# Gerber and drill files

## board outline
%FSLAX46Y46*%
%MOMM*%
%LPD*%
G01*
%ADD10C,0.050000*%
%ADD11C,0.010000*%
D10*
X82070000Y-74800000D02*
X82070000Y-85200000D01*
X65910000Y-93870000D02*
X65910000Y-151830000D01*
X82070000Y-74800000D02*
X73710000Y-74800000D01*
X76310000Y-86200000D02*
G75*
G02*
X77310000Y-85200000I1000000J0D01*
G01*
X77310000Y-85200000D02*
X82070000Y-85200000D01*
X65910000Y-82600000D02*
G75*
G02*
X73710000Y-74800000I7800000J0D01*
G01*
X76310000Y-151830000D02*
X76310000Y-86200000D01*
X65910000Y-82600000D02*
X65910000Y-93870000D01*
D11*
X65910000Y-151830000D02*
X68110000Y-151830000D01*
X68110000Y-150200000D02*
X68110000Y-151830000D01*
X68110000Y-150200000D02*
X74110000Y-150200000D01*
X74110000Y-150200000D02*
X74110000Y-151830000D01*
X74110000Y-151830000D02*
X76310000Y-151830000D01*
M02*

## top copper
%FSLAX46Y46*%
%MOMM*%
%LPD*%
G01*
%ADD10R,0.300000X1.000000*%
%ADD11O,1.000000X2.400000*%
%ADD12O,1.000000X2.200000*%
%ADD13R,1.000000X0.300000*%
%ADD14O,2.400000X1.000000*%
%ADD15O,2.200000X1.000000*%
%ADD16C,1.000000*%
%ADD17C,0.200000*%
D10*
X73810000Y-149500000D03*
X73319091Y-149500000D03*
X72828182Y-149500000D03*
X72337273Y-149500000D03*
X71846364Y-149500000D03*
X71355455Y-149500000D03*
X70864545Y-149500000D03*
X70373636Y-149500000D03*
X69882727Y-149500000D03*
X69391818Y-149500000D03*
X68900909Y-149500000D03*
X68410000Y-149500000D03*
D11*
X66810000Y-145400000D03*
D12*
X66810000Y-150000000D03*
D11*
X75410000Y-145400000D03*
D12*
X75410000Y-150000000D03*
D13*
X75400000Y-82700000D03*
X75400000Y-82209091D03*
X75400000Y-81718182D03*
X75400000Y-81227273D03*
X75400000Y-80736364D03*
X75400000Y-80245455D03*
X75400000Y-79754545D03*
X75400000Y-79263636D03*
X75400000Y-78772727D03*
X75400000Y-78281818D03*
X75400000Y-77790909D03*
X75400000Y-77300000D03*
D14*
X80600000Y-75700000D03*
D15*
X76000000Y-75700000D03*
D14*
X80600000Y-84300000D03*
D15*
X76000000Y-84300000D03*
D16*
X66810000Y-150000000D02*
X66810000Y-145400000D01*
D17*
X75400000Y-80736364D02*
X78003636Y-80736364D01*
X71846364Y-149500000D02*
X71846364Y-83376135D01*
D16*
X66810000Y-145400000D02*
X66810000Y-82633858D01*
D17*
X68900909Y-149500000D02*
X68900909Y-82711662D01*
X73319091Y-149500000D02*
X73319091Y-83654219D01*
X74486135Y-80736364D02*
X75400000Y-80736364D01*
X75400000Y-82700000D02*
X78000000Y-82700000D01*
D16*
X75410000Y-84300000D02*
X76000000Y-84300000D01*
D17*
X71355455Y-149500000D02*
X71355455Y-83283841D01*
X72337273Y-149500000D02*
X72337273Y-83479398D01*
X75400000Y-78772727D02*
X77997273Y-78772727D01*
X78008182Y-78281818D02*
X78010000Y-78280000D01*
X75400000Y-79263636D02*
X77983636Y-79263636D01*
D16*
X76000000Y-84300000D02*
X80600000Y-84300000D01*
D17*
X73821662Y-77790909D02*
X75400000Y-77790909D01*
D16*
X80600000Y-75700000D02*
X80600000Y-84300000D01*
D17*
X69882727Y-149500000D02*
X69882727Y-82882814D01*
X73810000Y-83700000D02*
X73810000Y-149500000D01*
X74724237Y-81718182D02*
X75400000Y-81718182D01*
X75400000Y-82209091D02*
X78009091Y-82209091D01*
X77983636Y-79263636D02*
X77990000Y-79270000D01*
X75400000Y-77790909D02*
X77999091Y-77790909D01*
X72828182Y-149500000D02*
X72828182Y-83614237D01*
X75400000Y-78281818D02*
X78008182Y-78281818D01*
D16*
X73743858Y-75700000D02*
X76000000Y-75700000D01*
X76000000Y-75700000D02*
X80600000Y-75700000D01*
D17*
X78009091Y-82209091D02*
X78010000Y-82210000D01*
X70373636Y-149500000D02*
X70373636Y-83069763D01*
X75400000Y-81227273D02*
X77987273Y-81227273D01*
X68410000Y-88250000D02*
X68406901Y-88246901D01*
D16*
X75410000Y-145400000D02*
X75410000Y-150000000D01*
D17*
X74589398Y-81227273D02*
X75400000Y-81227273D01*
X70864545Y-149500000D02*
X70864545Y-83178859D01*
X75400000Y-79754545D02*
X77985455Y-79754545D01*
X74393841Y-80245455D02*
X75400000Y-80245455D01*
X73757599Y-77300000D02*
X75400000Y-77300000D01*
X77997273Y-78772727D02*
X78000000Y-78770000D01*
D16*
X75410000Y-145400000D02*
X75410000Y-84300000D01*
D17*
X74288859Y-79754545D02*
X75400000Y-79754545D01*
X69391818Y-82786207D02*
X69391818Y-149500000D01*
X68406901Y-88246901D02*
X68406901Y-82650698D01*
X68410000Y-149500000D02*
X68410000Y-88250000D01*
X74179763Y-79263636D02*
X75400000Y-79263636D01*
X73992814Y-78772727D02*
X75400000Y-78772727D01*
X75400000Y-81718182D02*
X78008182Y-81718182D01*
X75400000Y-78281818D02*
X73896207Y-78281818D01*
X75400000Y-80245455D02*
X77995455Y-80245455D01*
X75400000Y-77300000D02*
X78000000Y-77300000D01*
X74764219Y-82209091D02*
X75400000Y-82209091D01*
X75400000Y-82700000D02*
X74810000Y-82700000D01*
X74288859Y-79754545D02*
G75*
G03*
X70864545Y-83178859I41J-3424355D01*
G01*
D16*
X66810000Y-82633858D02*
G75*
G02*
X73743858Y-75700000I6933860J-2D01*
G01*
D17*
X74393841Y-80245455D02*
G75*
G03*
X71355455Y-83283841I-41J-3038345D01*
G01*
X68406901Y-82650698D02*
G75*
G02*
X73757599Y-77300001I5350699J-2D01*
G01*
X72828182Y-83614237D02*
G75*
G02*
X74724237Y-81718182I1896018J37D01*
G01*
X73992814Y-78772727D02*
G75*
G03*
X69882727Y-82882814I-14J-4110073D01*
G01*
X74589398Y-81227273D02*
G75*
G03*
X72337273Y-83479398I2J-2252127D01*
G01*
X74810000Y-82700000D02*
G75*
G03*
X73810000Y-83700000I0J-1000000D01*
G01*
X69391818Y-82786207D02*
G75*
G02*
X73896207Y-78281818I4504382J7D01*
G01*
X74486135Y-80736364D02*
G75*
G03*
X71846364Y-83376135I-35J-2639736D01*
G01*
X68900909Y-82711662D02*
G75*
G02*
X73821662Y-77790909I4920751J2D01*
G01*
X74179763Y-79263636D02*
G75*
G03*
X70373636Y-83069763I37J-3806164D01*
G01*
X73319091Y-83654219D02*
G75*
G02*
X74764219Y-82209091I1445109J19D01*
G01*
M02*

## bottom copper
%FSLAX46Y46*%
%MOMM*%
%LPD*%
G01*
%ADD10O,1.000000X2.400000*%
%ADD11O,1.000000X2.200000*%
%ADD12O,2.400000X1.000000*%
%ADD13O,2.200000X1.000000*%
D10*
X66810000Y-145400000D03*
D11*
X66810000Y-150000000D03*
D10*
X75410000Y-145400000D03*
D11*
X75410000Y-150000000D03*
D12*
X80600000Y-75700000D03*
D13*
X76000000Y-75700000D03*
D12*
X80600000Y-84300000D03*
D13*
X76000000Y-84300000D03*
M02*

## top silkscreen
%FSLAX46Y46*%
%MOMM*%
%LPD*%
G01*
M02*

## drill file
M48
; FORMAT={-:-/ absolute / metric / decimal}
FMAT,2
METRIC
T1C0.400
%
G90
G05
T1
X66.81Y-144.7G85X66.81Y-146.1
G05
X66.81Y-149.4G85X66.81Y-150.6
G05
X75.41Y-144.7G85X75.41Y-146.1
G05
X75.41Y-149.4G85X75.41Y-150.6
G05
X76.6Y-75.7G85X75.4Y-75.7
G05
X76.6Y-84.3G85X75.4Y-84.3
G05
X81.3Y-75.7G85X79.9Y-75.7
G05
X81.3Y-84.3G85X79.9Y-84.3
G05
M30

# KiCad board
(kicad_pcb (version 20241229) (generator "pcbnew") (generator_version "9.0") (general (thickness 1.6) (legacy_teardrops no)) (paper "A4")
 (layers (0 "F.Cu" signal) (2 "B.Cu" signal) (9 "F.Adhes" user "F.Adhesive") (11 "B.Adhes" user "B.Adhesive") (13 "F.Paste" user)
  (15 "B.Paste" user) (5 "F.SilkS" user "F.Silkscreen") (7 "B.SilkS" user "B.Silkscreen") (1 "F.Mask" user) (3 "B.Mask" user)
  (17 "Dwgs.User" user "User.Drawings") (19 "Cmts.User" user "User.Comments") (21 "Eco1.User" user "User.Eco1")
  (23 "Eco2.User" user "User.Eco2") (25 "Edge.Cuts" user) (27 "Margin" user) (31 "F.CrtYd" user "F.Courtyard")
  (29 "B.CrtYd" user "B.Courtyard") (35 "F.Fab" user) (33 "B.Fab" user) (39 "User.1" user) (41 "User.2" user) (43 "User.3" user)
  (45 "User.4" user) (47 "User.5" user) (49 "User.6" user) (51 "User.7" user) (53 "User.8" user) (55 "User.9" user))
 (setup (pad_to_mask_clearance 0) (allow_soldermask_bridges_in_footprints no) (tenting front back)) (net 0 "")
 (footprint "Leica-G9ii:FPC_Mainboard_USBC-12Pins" (layer "F.Cu") (at 71.11 150)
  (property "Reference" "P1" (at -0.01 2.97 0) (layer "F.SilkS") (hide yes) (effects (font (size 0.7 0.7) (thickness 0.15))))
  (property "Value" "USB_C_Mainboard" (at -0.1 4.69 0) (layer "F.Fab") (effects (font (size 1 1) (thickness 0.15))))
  (fp_line (start -5.2 1.83) (end -3 1.83) (stroke (width 0.01) (type solid)) (layer "Edge.Cuts"))
  (fp_line (start -3 0.2) (end -3 1.83) (stroke (width 0.01) (type solid)) (layer "Edge.Cuts"))
  (fp_line (start -3 0.2) (end 3 0.2) (stroke (width 0.01) (type solid)) (layer "Edge.Cuts"))
  (fp_line (start 3 0.2) (end 3 1.83) (stroke (width 0.01) (type solid)) (layer "Edge.Cuts"))
  (fp_line (start 3 1.83) (end 5.2 1.83) (stroke (width 0.01) (type solid)) (layer "Edge.Cuts"))
  (pad "1" smd rect (at 2.7 -0.5) (size 0.3 1) (layers "F.Cu" "F.Mask" "F.Paste"))
  (pad "2" smd rect (at 2.209091 -0.5) (size 0.3 1) (layers "F.Cu" "F.Mask" "F.Paste"))
  (pad "3" smd rect (at 1.718182 -0.5) (size 0.3 1) (layers "F.Cu" "F.Mask" "F.Paste"))
  (pad "4" smd rect (at 1.227273 -0.5) (size 0.3 1) (layers "F.Cu" "F.Mask" "F.Paste"))
  (pad "5" smd rect (at 0.736364 -0.5) (size 0.3 1) (layers "F.Cu" "F.Mask" "F.Paste"))
  (pad "6" smd rect (at 0.245455 -0.5) (size 0.3 1) (layers "F.Cu" "F.Mask" "F.Paste"))
  (pad "7" smd rect (at -0.245455 -0.5) (size 0.3 1) (layers "F.Cu" "F.Mask" "F.Paste"))
  (pad "8" smd rect (at -0.736364 -0.5) (size 0.3 1) (layers "F.Cu" "F.Mask" "F.Paste"))
  (pad "9" smd rect (at -1.227273 -0.5) (size 0.3 1) (layers "F.Cu" "F.Mask" "F.Paste"))
  (pad "10" smd rect (at -1.718182 -0.5) (size 0.3 1) (layers "F.Cu" "F.Mask" "F.Paste"))
  (pad "11" smd rect (at -2.209091 -0.5) (size 0.3 1) (layers "F.Cu" "F.Mask" "F.Paste"))
  (pad "12" smd rect (at -2.7 -0.5) (size 0.3 1) (layers "F.Cu" "F.Mask" "F.Paste"))
  (pad "13" thru_hole oval (at -4.3 -4.6) (size 1 2.4) (drill oval 0.4 1.8) (layers "*.Cu" "*.Mask") (remove_unused_layers no))
  (pad "13" thru_hole oval (at -4.3 0) (size 1 2.2) (drill oval 0.4 1.6) (layers "*.Cu" "*.Mask") (remove_unused_layers no))
  (pad "13" thru_hole oval (at 4.3 -4.6) (size 1 2.4) (drill oval 0.4 1.8) (layers "*.Cu" "*.Mask") (remove_unused_layers no))
  (pad "13" thru_hole oval (at 4.3 0) (size 1 2.2) (drill oval 0.4 1.6) (layers "*.Cu" "*.Mask") (remove_unused_layers no)))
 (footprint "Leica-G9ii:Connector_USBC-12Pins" (layer "F.Cu") (at 76 80 -90)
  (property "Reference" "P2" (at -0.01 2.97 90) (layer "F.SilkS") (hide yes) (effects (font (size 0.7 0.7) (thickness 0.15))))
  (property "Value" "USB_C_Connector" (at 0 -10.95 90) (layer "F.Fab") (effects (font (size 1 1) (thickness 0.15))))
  (pad "1" smd rect (at 2.7 0.6 270) (size 0.3 1) (layers "F.Cu" "F.Mask" "F.Paste"))
  (pad "2" smd rect (at 2.209091 0.6 270) (size 0.3 1) (layers "F.Cu" "F.Mask" "F.Paste"))
  (pad "3" smd rect (at 1.718182 0.6 270) (size 0.3 1) (layers "F.Cu" "F.Mask" "F.Paste"))
  (pad "4" smd rect (at 1.227273 0.6 270) (size 0.3 1) (layers "F.Cu" "F.Mask" "F.Paste"))
  (pad "5" smd rect (at 0.736364 0.6 270) (size 0.3 1) (layers "F.Cu" "F.Mask" "F.Paste"))
  (pad "6" smd rect (at 0.245455 0.6 270) (size 0.3 1) (layers "F.Cu" "F.Mask" "F.Paste"))
  (pad "7" smd rect (at -0.245455 0.6 270) (size 0.3 1) (layers "F.Cu" "F.Mask" "F.Paste"))
  (pad "8" smd rect (at -0.736364 0.6 270) (size 0.3 1) (layers "F.Cu" "F.Mask" "F.Paste"))
  (pad "9" smd rect (at -1.227273 0.6 270) (size 0.3 1) (layers "F.Cu" "F.Mask" "F.Paste"))
  (pad "10" smd rect (at -1.718182 0.6 270) (size 0.3 1) (layers "F.Cu" "F.Mask" "F.Paste"))
  (pad "11" smd rect (at -2.209091 0.6 270) (size 0.3 1) (layers "F.Cu" "F.Mask" "F.Paste"))
  (pad "12" smd rect (at -2.7 0.6 270) (size 0.3 1) (layers "F.Cu" "F.Mask" "F.Paste"))
  (pad "13" thru_hole oval (at -4.3 -4.6 270) (size 1 2.4) (drill oval 0.4 1.8) (layers "*.Cu" "*.Mask") (remove_unused_layers no))
  (pad "13" thru_hole oval (at -4.3 0 270) (size 1 2.2) (drill oval 0.4 1.6) (layers "*.Cu" "*.Mask") (remove_unused_layers no))
  (pad "13" thru_hole oval (at 4.3 -4.6 270) (size 1 2.4) (drill oval 0.4 1.8) (layers "*.Cu" "*.Mask") (remove_unused_layers no))
  (pad "13" thru_hole oval (at 4.3 0 270) (size 1 2.2) (drill oval 0.4 1.6) (layers "*.Cu" "*.Mask") (remove_unused_layers no)))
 (gr_line (start 82.07 74.8) (end 82.07 85.2) (stroke (width 0.05) (type solid)) (layer "Edge.Cuts"))
 (gr_line (start 65.91 93.87) (end 65.91 151.83) (stroke (width 0.05) (type solid)) (layer "Edge.Cuts"))
 (gr_line (start 82.07 74.8) (end 73.71 74.8) (stroke (width 0.05) (type solid)) (layer "Edge.Cuts"))
 (gr_arc (start 76.31 86.2) (mid 76.602893 85.492893) (end 77.31 85.2) (stroke (width 0.05) (type default)) (layer "Edge.Cuts"))
 (gr_line (start 77.31 85.2) (end 82.07 85.2) (stroke (width 0.05) (type default)) (layer "Edge.Cuts"))
 (gr_arc (start 65.91 82.6) (mid 68.194567 77.084567) (end 73.71 74.8) (stroke (width 0.05) (type default)) (layer "Edge.Cuts"))
 (gr_line (start 76.31 151.83) (end 76.31 86.2) (stroke (width 0.05) (type solid)) (layer "Edge.Cuts"))
 (gr_line (start 65.91 82.6) (end 65.91 93.87) (stroke (width 0.05) (type solid)) (layer "Edge.Cuts"))
 (segment (start 66.81 150) (end 66.81 145.4) (width 1) (layer "F.Cu") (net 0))
 (segment (start 75.4 80.736364) (end 78.003636 80.736364) (width 0.2) (layer "F.Cu") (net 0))
 (segment (start 71.846364 149.5) (end 71.846364 83.376135) (width 0.2) (layer "F.Cu") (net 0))
 (segment (start 66.81 145.4) (end 66.81 82.633858) (width 1) (layer "F.Cu") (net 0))
 (segment (start 68.900909 149.5) (end 68.900909 82.711662) (width 0.2) (layer "F.Cu") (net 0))
 (segment (start 73.319091 149.5) (end 73.319091 83.654219) (width 0.2) (layer "F.Cu") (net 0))
 (segment (start 74.486135 80.736364) (end 75.4 80.736364) (width 0.2) (layer "F.Cu") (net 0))
 (segment (start 75.4 82.7) (end 78 82.7) (width 0.2) (layer "F.Cu") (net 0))
 (segment (start 75.41 84.3) (end 76 84.3) (width 1) (layer "F.Cu") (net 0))
 (segment (start 71.355455 149.5) (end 71.355455 83.283841) (width 0.2) (layer "F.Cu") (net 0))
 (segment (start 72.337273 149.5) (end 72.337273 83.479398) (width 0.2) (layer "F.Cu") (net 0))
 (segment (start 75.4 78.772727) (end 77.997273 78.772727) (width 0.2) (layer "F.Cu") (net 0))
 (segment (start 78.008182 78.281818) (end 78.01 78.28) (width 0.2) (layer "F.Cu") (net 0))
 (segment (start 75.4 79.263636) (end 77.983636 79.263636) (width 0.2) (layer "F.Cu") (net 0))
 (segment (start 76 84.3) (end 80.6 84.3) (width 1) (layer "F.Cu") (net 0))
 (segment (start 73.821662 77.790909) (end 75.4 77.790909) (width 0.2) (layer "F.Cu") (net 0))
 (segment (start 80.6 75.7) (end 80.6 84.3) (width 1) (layer "F.Cu") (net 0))
 (segment (start 69.882727 149.5) (end 69.882727 82.882814) (width 0.2) (layer "F.Cu") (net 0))
 (segment (start 73.81 83.7) (end 73.81 149.5) (width 0.2) (layer "F.Cu") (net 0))
 (segment (start 74.724237 81.718182) (end 75.4 81.718182) (width 0.2) (layer "F.Cu") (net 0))
 (segment (start 75.4 82.209091) (end 78.009091 82.209091) (width 0.2) (layer "F.Cu") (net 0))
 (segment (start 77.983636 79.263636) (end 77.99 79.27) (width 0.2) (layer "F.Cu") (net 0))
 (segment (start 75.4 77.790909) (end 77.999091 77.790909) (width 0.2) (layer "F.Cu") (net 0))
 (segment (start 72.828182 149.5) (end 72.828182 83.614237) (width 0.2) (layer "F.Cu") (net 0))
 (segment (start 75.4 78.281818) (end 78.008182 78.281818) (width 0.2) (layer "F.Cu") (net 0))
 (segment (start 73.743858 75.7) (end 76 75.7) (width 1) (layer "F.Cu") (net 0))
 (segment (start 76 75.7) (end 80.6 75.7) (width 1) (layer "F.Cu") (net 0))
 (segment (start 78.009091 82.209091) (end 78.01 82.21) (width 0.2) (layer "F.Cu") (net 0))
 (segment (start 70.373636 149.5) (end 70.373636 83.069763) (width 0.2) (layer "F.Cu") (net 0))
 (segment (start 75.4 81.227273) (end 77.987273 81.227273) (width 0.2) (layer "F.Cu") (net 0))
 (segment (start 68.41 88.25) (end 68.406901 88.246901) (width 0.2) (layer "F.Cu") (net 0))
 (segment (start 75.41 145.4) (end 75.41 150) (width 1) (layer "F.Cu") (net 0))
 (segment (start 74.589398 81.227273) (end 75.4 81.227273) (width 0.2) (layer "F.Cu") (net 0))
 (segment (start 70.864545 149.5) (end 70.864545 83.178859) (width 0.2) (layer "F.Cu") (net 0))
 (segment (start 75.4 79.754545) (end 77.985455 79.754545) (width 0.2) (layer "F.Cu") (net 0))
 (segment (start 74.393841 80.245455) (end 75.4 80.245455) (width 0.2) (layer "F.Cu") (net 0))
 (segment (start 73.757599 77.3) (end 75.4 77.3) (width 0.2) (layer "F.Cu") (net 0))
 (segment (start 77.997273 78.772727) (end 78 78.77) (width 0.2) (layer "F.Cu") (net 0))
 (segment (start 75.41 145.4) (end 75.41 84.3) (width 1) (layer "F.Cu") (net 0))
 (segment (start 74.288859 79.754545) (end 75.4 79.754545) (width 0.2) (layer "F.Cu") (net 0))
 (segment (start 69.391818 82.786207) (end 69.391818 149.5) (width 0.2) (layer "F.Cu") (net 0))
 (segment (start 68.406901 88.246901) (end 68.406901 82.650698) (width 0.2) (layer "F.Cu") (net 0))
 (segment (start 68.41 149.5) (end 68.41 88.25) (width 0.2) (layer "F.Cu") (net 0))
 (segment (start 74.179763 79.263636) (end 75.4 79.263636) (width 0.2) (layer "F.Cu") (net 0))
 (segment (start 73.992814 78.772727) (end 75.4 78.772727) (width 0.2) (layer "F.Cu") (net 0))
 (segment (start 75.4 81.718182) (end 78.008182 81.718182) (width 0.2) (layer "F.Cu") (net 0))
 (segment (start 75.4 78.281818) (end 73.896207 78.281818) (width 0.2) (layer "F.Cu") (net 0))
 (segment (start 75.4 80.245455) (end 77.995455 80.245455) (width 0.2) (layer "F.Cu") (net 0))
 (segment (start 75.4 77.3) (end 78 77.3) (width 0.2) (layer "F.Cu") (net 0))
 (segment (start 74.764219 82.209091) (end 75.4 82.209091) (width 0.2) (layer "F.Cu") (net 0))
 (segment (start 75.4 82.7) (end 74.81 82.7) (width 0.2) (layer "F.Cu") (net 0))
 (arc (start 74.288859 79.754545) (mid 71.867503 80.757503) (end 70.864545 83.178859) (width 0.2) (layer "F.Cu") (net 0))
 (arc (start 66.81 82.633858) (mid 68.84088 77.73088) (end 73.743858 75.7) (width 1) (layer "F.Cu") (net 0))
 (arc (start 74.393841 80.245455) (mid 72.245378 81.135378) (end 71.355455 83.283841) (width 0.2) (layer "F.Cu") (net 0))
 (arc (start 68.406901 82.650698) (mid 69.974084 78.867183) (end 73.757599 77.3) (width 0.2) (layer "F.Cu") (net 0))
 (arc (start 72.828182 83.614237) (mid 73.383524 82.273524) (end 74.724237 81.718182) (width 0.2) (layer "F.Cu") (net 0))
 (arc (start 73.992814 78.772727) (mid 71.086544 79.976544) (end 69.882727 82.882814) (width 0.2) (layer "F.Cu") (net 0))
 (arc (start 74.589398 81.227273) (mid 72.996905 81.886905) (end 72.337273 83.479398) (width 0.2) (layer "F.Cu") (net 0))
 (arc (start 74.81 82.7) (mid 74.102893 82.992893) (end 73.81 83.7) (width 0.2) (layer "F.Cu") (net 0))
 (arc (start 69.391818 82.786207) (mid 70.711123 79.601123) (end 73.896207 78.281818) (width 0.2) (layer "F.Cu") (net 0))
 (arc (start 74.486135 80.736364) (mid 72.619535 81.509535) (end 71.846364 83.376135) (width 0.2) (layer "F.Cu") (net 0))
 (arc (start 68.900909 82.711662) (mid 70.342164 79.232164) (end 73.821662 77.790909) (width 0.2) (layer "F.Cu") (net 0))
 (arc (start 74.179763 79.263636) (mid 71.488425 80.378425) (end 70.373636 83.069763) (width 0.2) (layer "F.Cu") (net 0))
 (arc (start 73.319091 83.654219) (mid 73.742359 82.632359) (end 74.764219 82.209091) (width 0.2) (layer "F.Cu") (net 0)))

